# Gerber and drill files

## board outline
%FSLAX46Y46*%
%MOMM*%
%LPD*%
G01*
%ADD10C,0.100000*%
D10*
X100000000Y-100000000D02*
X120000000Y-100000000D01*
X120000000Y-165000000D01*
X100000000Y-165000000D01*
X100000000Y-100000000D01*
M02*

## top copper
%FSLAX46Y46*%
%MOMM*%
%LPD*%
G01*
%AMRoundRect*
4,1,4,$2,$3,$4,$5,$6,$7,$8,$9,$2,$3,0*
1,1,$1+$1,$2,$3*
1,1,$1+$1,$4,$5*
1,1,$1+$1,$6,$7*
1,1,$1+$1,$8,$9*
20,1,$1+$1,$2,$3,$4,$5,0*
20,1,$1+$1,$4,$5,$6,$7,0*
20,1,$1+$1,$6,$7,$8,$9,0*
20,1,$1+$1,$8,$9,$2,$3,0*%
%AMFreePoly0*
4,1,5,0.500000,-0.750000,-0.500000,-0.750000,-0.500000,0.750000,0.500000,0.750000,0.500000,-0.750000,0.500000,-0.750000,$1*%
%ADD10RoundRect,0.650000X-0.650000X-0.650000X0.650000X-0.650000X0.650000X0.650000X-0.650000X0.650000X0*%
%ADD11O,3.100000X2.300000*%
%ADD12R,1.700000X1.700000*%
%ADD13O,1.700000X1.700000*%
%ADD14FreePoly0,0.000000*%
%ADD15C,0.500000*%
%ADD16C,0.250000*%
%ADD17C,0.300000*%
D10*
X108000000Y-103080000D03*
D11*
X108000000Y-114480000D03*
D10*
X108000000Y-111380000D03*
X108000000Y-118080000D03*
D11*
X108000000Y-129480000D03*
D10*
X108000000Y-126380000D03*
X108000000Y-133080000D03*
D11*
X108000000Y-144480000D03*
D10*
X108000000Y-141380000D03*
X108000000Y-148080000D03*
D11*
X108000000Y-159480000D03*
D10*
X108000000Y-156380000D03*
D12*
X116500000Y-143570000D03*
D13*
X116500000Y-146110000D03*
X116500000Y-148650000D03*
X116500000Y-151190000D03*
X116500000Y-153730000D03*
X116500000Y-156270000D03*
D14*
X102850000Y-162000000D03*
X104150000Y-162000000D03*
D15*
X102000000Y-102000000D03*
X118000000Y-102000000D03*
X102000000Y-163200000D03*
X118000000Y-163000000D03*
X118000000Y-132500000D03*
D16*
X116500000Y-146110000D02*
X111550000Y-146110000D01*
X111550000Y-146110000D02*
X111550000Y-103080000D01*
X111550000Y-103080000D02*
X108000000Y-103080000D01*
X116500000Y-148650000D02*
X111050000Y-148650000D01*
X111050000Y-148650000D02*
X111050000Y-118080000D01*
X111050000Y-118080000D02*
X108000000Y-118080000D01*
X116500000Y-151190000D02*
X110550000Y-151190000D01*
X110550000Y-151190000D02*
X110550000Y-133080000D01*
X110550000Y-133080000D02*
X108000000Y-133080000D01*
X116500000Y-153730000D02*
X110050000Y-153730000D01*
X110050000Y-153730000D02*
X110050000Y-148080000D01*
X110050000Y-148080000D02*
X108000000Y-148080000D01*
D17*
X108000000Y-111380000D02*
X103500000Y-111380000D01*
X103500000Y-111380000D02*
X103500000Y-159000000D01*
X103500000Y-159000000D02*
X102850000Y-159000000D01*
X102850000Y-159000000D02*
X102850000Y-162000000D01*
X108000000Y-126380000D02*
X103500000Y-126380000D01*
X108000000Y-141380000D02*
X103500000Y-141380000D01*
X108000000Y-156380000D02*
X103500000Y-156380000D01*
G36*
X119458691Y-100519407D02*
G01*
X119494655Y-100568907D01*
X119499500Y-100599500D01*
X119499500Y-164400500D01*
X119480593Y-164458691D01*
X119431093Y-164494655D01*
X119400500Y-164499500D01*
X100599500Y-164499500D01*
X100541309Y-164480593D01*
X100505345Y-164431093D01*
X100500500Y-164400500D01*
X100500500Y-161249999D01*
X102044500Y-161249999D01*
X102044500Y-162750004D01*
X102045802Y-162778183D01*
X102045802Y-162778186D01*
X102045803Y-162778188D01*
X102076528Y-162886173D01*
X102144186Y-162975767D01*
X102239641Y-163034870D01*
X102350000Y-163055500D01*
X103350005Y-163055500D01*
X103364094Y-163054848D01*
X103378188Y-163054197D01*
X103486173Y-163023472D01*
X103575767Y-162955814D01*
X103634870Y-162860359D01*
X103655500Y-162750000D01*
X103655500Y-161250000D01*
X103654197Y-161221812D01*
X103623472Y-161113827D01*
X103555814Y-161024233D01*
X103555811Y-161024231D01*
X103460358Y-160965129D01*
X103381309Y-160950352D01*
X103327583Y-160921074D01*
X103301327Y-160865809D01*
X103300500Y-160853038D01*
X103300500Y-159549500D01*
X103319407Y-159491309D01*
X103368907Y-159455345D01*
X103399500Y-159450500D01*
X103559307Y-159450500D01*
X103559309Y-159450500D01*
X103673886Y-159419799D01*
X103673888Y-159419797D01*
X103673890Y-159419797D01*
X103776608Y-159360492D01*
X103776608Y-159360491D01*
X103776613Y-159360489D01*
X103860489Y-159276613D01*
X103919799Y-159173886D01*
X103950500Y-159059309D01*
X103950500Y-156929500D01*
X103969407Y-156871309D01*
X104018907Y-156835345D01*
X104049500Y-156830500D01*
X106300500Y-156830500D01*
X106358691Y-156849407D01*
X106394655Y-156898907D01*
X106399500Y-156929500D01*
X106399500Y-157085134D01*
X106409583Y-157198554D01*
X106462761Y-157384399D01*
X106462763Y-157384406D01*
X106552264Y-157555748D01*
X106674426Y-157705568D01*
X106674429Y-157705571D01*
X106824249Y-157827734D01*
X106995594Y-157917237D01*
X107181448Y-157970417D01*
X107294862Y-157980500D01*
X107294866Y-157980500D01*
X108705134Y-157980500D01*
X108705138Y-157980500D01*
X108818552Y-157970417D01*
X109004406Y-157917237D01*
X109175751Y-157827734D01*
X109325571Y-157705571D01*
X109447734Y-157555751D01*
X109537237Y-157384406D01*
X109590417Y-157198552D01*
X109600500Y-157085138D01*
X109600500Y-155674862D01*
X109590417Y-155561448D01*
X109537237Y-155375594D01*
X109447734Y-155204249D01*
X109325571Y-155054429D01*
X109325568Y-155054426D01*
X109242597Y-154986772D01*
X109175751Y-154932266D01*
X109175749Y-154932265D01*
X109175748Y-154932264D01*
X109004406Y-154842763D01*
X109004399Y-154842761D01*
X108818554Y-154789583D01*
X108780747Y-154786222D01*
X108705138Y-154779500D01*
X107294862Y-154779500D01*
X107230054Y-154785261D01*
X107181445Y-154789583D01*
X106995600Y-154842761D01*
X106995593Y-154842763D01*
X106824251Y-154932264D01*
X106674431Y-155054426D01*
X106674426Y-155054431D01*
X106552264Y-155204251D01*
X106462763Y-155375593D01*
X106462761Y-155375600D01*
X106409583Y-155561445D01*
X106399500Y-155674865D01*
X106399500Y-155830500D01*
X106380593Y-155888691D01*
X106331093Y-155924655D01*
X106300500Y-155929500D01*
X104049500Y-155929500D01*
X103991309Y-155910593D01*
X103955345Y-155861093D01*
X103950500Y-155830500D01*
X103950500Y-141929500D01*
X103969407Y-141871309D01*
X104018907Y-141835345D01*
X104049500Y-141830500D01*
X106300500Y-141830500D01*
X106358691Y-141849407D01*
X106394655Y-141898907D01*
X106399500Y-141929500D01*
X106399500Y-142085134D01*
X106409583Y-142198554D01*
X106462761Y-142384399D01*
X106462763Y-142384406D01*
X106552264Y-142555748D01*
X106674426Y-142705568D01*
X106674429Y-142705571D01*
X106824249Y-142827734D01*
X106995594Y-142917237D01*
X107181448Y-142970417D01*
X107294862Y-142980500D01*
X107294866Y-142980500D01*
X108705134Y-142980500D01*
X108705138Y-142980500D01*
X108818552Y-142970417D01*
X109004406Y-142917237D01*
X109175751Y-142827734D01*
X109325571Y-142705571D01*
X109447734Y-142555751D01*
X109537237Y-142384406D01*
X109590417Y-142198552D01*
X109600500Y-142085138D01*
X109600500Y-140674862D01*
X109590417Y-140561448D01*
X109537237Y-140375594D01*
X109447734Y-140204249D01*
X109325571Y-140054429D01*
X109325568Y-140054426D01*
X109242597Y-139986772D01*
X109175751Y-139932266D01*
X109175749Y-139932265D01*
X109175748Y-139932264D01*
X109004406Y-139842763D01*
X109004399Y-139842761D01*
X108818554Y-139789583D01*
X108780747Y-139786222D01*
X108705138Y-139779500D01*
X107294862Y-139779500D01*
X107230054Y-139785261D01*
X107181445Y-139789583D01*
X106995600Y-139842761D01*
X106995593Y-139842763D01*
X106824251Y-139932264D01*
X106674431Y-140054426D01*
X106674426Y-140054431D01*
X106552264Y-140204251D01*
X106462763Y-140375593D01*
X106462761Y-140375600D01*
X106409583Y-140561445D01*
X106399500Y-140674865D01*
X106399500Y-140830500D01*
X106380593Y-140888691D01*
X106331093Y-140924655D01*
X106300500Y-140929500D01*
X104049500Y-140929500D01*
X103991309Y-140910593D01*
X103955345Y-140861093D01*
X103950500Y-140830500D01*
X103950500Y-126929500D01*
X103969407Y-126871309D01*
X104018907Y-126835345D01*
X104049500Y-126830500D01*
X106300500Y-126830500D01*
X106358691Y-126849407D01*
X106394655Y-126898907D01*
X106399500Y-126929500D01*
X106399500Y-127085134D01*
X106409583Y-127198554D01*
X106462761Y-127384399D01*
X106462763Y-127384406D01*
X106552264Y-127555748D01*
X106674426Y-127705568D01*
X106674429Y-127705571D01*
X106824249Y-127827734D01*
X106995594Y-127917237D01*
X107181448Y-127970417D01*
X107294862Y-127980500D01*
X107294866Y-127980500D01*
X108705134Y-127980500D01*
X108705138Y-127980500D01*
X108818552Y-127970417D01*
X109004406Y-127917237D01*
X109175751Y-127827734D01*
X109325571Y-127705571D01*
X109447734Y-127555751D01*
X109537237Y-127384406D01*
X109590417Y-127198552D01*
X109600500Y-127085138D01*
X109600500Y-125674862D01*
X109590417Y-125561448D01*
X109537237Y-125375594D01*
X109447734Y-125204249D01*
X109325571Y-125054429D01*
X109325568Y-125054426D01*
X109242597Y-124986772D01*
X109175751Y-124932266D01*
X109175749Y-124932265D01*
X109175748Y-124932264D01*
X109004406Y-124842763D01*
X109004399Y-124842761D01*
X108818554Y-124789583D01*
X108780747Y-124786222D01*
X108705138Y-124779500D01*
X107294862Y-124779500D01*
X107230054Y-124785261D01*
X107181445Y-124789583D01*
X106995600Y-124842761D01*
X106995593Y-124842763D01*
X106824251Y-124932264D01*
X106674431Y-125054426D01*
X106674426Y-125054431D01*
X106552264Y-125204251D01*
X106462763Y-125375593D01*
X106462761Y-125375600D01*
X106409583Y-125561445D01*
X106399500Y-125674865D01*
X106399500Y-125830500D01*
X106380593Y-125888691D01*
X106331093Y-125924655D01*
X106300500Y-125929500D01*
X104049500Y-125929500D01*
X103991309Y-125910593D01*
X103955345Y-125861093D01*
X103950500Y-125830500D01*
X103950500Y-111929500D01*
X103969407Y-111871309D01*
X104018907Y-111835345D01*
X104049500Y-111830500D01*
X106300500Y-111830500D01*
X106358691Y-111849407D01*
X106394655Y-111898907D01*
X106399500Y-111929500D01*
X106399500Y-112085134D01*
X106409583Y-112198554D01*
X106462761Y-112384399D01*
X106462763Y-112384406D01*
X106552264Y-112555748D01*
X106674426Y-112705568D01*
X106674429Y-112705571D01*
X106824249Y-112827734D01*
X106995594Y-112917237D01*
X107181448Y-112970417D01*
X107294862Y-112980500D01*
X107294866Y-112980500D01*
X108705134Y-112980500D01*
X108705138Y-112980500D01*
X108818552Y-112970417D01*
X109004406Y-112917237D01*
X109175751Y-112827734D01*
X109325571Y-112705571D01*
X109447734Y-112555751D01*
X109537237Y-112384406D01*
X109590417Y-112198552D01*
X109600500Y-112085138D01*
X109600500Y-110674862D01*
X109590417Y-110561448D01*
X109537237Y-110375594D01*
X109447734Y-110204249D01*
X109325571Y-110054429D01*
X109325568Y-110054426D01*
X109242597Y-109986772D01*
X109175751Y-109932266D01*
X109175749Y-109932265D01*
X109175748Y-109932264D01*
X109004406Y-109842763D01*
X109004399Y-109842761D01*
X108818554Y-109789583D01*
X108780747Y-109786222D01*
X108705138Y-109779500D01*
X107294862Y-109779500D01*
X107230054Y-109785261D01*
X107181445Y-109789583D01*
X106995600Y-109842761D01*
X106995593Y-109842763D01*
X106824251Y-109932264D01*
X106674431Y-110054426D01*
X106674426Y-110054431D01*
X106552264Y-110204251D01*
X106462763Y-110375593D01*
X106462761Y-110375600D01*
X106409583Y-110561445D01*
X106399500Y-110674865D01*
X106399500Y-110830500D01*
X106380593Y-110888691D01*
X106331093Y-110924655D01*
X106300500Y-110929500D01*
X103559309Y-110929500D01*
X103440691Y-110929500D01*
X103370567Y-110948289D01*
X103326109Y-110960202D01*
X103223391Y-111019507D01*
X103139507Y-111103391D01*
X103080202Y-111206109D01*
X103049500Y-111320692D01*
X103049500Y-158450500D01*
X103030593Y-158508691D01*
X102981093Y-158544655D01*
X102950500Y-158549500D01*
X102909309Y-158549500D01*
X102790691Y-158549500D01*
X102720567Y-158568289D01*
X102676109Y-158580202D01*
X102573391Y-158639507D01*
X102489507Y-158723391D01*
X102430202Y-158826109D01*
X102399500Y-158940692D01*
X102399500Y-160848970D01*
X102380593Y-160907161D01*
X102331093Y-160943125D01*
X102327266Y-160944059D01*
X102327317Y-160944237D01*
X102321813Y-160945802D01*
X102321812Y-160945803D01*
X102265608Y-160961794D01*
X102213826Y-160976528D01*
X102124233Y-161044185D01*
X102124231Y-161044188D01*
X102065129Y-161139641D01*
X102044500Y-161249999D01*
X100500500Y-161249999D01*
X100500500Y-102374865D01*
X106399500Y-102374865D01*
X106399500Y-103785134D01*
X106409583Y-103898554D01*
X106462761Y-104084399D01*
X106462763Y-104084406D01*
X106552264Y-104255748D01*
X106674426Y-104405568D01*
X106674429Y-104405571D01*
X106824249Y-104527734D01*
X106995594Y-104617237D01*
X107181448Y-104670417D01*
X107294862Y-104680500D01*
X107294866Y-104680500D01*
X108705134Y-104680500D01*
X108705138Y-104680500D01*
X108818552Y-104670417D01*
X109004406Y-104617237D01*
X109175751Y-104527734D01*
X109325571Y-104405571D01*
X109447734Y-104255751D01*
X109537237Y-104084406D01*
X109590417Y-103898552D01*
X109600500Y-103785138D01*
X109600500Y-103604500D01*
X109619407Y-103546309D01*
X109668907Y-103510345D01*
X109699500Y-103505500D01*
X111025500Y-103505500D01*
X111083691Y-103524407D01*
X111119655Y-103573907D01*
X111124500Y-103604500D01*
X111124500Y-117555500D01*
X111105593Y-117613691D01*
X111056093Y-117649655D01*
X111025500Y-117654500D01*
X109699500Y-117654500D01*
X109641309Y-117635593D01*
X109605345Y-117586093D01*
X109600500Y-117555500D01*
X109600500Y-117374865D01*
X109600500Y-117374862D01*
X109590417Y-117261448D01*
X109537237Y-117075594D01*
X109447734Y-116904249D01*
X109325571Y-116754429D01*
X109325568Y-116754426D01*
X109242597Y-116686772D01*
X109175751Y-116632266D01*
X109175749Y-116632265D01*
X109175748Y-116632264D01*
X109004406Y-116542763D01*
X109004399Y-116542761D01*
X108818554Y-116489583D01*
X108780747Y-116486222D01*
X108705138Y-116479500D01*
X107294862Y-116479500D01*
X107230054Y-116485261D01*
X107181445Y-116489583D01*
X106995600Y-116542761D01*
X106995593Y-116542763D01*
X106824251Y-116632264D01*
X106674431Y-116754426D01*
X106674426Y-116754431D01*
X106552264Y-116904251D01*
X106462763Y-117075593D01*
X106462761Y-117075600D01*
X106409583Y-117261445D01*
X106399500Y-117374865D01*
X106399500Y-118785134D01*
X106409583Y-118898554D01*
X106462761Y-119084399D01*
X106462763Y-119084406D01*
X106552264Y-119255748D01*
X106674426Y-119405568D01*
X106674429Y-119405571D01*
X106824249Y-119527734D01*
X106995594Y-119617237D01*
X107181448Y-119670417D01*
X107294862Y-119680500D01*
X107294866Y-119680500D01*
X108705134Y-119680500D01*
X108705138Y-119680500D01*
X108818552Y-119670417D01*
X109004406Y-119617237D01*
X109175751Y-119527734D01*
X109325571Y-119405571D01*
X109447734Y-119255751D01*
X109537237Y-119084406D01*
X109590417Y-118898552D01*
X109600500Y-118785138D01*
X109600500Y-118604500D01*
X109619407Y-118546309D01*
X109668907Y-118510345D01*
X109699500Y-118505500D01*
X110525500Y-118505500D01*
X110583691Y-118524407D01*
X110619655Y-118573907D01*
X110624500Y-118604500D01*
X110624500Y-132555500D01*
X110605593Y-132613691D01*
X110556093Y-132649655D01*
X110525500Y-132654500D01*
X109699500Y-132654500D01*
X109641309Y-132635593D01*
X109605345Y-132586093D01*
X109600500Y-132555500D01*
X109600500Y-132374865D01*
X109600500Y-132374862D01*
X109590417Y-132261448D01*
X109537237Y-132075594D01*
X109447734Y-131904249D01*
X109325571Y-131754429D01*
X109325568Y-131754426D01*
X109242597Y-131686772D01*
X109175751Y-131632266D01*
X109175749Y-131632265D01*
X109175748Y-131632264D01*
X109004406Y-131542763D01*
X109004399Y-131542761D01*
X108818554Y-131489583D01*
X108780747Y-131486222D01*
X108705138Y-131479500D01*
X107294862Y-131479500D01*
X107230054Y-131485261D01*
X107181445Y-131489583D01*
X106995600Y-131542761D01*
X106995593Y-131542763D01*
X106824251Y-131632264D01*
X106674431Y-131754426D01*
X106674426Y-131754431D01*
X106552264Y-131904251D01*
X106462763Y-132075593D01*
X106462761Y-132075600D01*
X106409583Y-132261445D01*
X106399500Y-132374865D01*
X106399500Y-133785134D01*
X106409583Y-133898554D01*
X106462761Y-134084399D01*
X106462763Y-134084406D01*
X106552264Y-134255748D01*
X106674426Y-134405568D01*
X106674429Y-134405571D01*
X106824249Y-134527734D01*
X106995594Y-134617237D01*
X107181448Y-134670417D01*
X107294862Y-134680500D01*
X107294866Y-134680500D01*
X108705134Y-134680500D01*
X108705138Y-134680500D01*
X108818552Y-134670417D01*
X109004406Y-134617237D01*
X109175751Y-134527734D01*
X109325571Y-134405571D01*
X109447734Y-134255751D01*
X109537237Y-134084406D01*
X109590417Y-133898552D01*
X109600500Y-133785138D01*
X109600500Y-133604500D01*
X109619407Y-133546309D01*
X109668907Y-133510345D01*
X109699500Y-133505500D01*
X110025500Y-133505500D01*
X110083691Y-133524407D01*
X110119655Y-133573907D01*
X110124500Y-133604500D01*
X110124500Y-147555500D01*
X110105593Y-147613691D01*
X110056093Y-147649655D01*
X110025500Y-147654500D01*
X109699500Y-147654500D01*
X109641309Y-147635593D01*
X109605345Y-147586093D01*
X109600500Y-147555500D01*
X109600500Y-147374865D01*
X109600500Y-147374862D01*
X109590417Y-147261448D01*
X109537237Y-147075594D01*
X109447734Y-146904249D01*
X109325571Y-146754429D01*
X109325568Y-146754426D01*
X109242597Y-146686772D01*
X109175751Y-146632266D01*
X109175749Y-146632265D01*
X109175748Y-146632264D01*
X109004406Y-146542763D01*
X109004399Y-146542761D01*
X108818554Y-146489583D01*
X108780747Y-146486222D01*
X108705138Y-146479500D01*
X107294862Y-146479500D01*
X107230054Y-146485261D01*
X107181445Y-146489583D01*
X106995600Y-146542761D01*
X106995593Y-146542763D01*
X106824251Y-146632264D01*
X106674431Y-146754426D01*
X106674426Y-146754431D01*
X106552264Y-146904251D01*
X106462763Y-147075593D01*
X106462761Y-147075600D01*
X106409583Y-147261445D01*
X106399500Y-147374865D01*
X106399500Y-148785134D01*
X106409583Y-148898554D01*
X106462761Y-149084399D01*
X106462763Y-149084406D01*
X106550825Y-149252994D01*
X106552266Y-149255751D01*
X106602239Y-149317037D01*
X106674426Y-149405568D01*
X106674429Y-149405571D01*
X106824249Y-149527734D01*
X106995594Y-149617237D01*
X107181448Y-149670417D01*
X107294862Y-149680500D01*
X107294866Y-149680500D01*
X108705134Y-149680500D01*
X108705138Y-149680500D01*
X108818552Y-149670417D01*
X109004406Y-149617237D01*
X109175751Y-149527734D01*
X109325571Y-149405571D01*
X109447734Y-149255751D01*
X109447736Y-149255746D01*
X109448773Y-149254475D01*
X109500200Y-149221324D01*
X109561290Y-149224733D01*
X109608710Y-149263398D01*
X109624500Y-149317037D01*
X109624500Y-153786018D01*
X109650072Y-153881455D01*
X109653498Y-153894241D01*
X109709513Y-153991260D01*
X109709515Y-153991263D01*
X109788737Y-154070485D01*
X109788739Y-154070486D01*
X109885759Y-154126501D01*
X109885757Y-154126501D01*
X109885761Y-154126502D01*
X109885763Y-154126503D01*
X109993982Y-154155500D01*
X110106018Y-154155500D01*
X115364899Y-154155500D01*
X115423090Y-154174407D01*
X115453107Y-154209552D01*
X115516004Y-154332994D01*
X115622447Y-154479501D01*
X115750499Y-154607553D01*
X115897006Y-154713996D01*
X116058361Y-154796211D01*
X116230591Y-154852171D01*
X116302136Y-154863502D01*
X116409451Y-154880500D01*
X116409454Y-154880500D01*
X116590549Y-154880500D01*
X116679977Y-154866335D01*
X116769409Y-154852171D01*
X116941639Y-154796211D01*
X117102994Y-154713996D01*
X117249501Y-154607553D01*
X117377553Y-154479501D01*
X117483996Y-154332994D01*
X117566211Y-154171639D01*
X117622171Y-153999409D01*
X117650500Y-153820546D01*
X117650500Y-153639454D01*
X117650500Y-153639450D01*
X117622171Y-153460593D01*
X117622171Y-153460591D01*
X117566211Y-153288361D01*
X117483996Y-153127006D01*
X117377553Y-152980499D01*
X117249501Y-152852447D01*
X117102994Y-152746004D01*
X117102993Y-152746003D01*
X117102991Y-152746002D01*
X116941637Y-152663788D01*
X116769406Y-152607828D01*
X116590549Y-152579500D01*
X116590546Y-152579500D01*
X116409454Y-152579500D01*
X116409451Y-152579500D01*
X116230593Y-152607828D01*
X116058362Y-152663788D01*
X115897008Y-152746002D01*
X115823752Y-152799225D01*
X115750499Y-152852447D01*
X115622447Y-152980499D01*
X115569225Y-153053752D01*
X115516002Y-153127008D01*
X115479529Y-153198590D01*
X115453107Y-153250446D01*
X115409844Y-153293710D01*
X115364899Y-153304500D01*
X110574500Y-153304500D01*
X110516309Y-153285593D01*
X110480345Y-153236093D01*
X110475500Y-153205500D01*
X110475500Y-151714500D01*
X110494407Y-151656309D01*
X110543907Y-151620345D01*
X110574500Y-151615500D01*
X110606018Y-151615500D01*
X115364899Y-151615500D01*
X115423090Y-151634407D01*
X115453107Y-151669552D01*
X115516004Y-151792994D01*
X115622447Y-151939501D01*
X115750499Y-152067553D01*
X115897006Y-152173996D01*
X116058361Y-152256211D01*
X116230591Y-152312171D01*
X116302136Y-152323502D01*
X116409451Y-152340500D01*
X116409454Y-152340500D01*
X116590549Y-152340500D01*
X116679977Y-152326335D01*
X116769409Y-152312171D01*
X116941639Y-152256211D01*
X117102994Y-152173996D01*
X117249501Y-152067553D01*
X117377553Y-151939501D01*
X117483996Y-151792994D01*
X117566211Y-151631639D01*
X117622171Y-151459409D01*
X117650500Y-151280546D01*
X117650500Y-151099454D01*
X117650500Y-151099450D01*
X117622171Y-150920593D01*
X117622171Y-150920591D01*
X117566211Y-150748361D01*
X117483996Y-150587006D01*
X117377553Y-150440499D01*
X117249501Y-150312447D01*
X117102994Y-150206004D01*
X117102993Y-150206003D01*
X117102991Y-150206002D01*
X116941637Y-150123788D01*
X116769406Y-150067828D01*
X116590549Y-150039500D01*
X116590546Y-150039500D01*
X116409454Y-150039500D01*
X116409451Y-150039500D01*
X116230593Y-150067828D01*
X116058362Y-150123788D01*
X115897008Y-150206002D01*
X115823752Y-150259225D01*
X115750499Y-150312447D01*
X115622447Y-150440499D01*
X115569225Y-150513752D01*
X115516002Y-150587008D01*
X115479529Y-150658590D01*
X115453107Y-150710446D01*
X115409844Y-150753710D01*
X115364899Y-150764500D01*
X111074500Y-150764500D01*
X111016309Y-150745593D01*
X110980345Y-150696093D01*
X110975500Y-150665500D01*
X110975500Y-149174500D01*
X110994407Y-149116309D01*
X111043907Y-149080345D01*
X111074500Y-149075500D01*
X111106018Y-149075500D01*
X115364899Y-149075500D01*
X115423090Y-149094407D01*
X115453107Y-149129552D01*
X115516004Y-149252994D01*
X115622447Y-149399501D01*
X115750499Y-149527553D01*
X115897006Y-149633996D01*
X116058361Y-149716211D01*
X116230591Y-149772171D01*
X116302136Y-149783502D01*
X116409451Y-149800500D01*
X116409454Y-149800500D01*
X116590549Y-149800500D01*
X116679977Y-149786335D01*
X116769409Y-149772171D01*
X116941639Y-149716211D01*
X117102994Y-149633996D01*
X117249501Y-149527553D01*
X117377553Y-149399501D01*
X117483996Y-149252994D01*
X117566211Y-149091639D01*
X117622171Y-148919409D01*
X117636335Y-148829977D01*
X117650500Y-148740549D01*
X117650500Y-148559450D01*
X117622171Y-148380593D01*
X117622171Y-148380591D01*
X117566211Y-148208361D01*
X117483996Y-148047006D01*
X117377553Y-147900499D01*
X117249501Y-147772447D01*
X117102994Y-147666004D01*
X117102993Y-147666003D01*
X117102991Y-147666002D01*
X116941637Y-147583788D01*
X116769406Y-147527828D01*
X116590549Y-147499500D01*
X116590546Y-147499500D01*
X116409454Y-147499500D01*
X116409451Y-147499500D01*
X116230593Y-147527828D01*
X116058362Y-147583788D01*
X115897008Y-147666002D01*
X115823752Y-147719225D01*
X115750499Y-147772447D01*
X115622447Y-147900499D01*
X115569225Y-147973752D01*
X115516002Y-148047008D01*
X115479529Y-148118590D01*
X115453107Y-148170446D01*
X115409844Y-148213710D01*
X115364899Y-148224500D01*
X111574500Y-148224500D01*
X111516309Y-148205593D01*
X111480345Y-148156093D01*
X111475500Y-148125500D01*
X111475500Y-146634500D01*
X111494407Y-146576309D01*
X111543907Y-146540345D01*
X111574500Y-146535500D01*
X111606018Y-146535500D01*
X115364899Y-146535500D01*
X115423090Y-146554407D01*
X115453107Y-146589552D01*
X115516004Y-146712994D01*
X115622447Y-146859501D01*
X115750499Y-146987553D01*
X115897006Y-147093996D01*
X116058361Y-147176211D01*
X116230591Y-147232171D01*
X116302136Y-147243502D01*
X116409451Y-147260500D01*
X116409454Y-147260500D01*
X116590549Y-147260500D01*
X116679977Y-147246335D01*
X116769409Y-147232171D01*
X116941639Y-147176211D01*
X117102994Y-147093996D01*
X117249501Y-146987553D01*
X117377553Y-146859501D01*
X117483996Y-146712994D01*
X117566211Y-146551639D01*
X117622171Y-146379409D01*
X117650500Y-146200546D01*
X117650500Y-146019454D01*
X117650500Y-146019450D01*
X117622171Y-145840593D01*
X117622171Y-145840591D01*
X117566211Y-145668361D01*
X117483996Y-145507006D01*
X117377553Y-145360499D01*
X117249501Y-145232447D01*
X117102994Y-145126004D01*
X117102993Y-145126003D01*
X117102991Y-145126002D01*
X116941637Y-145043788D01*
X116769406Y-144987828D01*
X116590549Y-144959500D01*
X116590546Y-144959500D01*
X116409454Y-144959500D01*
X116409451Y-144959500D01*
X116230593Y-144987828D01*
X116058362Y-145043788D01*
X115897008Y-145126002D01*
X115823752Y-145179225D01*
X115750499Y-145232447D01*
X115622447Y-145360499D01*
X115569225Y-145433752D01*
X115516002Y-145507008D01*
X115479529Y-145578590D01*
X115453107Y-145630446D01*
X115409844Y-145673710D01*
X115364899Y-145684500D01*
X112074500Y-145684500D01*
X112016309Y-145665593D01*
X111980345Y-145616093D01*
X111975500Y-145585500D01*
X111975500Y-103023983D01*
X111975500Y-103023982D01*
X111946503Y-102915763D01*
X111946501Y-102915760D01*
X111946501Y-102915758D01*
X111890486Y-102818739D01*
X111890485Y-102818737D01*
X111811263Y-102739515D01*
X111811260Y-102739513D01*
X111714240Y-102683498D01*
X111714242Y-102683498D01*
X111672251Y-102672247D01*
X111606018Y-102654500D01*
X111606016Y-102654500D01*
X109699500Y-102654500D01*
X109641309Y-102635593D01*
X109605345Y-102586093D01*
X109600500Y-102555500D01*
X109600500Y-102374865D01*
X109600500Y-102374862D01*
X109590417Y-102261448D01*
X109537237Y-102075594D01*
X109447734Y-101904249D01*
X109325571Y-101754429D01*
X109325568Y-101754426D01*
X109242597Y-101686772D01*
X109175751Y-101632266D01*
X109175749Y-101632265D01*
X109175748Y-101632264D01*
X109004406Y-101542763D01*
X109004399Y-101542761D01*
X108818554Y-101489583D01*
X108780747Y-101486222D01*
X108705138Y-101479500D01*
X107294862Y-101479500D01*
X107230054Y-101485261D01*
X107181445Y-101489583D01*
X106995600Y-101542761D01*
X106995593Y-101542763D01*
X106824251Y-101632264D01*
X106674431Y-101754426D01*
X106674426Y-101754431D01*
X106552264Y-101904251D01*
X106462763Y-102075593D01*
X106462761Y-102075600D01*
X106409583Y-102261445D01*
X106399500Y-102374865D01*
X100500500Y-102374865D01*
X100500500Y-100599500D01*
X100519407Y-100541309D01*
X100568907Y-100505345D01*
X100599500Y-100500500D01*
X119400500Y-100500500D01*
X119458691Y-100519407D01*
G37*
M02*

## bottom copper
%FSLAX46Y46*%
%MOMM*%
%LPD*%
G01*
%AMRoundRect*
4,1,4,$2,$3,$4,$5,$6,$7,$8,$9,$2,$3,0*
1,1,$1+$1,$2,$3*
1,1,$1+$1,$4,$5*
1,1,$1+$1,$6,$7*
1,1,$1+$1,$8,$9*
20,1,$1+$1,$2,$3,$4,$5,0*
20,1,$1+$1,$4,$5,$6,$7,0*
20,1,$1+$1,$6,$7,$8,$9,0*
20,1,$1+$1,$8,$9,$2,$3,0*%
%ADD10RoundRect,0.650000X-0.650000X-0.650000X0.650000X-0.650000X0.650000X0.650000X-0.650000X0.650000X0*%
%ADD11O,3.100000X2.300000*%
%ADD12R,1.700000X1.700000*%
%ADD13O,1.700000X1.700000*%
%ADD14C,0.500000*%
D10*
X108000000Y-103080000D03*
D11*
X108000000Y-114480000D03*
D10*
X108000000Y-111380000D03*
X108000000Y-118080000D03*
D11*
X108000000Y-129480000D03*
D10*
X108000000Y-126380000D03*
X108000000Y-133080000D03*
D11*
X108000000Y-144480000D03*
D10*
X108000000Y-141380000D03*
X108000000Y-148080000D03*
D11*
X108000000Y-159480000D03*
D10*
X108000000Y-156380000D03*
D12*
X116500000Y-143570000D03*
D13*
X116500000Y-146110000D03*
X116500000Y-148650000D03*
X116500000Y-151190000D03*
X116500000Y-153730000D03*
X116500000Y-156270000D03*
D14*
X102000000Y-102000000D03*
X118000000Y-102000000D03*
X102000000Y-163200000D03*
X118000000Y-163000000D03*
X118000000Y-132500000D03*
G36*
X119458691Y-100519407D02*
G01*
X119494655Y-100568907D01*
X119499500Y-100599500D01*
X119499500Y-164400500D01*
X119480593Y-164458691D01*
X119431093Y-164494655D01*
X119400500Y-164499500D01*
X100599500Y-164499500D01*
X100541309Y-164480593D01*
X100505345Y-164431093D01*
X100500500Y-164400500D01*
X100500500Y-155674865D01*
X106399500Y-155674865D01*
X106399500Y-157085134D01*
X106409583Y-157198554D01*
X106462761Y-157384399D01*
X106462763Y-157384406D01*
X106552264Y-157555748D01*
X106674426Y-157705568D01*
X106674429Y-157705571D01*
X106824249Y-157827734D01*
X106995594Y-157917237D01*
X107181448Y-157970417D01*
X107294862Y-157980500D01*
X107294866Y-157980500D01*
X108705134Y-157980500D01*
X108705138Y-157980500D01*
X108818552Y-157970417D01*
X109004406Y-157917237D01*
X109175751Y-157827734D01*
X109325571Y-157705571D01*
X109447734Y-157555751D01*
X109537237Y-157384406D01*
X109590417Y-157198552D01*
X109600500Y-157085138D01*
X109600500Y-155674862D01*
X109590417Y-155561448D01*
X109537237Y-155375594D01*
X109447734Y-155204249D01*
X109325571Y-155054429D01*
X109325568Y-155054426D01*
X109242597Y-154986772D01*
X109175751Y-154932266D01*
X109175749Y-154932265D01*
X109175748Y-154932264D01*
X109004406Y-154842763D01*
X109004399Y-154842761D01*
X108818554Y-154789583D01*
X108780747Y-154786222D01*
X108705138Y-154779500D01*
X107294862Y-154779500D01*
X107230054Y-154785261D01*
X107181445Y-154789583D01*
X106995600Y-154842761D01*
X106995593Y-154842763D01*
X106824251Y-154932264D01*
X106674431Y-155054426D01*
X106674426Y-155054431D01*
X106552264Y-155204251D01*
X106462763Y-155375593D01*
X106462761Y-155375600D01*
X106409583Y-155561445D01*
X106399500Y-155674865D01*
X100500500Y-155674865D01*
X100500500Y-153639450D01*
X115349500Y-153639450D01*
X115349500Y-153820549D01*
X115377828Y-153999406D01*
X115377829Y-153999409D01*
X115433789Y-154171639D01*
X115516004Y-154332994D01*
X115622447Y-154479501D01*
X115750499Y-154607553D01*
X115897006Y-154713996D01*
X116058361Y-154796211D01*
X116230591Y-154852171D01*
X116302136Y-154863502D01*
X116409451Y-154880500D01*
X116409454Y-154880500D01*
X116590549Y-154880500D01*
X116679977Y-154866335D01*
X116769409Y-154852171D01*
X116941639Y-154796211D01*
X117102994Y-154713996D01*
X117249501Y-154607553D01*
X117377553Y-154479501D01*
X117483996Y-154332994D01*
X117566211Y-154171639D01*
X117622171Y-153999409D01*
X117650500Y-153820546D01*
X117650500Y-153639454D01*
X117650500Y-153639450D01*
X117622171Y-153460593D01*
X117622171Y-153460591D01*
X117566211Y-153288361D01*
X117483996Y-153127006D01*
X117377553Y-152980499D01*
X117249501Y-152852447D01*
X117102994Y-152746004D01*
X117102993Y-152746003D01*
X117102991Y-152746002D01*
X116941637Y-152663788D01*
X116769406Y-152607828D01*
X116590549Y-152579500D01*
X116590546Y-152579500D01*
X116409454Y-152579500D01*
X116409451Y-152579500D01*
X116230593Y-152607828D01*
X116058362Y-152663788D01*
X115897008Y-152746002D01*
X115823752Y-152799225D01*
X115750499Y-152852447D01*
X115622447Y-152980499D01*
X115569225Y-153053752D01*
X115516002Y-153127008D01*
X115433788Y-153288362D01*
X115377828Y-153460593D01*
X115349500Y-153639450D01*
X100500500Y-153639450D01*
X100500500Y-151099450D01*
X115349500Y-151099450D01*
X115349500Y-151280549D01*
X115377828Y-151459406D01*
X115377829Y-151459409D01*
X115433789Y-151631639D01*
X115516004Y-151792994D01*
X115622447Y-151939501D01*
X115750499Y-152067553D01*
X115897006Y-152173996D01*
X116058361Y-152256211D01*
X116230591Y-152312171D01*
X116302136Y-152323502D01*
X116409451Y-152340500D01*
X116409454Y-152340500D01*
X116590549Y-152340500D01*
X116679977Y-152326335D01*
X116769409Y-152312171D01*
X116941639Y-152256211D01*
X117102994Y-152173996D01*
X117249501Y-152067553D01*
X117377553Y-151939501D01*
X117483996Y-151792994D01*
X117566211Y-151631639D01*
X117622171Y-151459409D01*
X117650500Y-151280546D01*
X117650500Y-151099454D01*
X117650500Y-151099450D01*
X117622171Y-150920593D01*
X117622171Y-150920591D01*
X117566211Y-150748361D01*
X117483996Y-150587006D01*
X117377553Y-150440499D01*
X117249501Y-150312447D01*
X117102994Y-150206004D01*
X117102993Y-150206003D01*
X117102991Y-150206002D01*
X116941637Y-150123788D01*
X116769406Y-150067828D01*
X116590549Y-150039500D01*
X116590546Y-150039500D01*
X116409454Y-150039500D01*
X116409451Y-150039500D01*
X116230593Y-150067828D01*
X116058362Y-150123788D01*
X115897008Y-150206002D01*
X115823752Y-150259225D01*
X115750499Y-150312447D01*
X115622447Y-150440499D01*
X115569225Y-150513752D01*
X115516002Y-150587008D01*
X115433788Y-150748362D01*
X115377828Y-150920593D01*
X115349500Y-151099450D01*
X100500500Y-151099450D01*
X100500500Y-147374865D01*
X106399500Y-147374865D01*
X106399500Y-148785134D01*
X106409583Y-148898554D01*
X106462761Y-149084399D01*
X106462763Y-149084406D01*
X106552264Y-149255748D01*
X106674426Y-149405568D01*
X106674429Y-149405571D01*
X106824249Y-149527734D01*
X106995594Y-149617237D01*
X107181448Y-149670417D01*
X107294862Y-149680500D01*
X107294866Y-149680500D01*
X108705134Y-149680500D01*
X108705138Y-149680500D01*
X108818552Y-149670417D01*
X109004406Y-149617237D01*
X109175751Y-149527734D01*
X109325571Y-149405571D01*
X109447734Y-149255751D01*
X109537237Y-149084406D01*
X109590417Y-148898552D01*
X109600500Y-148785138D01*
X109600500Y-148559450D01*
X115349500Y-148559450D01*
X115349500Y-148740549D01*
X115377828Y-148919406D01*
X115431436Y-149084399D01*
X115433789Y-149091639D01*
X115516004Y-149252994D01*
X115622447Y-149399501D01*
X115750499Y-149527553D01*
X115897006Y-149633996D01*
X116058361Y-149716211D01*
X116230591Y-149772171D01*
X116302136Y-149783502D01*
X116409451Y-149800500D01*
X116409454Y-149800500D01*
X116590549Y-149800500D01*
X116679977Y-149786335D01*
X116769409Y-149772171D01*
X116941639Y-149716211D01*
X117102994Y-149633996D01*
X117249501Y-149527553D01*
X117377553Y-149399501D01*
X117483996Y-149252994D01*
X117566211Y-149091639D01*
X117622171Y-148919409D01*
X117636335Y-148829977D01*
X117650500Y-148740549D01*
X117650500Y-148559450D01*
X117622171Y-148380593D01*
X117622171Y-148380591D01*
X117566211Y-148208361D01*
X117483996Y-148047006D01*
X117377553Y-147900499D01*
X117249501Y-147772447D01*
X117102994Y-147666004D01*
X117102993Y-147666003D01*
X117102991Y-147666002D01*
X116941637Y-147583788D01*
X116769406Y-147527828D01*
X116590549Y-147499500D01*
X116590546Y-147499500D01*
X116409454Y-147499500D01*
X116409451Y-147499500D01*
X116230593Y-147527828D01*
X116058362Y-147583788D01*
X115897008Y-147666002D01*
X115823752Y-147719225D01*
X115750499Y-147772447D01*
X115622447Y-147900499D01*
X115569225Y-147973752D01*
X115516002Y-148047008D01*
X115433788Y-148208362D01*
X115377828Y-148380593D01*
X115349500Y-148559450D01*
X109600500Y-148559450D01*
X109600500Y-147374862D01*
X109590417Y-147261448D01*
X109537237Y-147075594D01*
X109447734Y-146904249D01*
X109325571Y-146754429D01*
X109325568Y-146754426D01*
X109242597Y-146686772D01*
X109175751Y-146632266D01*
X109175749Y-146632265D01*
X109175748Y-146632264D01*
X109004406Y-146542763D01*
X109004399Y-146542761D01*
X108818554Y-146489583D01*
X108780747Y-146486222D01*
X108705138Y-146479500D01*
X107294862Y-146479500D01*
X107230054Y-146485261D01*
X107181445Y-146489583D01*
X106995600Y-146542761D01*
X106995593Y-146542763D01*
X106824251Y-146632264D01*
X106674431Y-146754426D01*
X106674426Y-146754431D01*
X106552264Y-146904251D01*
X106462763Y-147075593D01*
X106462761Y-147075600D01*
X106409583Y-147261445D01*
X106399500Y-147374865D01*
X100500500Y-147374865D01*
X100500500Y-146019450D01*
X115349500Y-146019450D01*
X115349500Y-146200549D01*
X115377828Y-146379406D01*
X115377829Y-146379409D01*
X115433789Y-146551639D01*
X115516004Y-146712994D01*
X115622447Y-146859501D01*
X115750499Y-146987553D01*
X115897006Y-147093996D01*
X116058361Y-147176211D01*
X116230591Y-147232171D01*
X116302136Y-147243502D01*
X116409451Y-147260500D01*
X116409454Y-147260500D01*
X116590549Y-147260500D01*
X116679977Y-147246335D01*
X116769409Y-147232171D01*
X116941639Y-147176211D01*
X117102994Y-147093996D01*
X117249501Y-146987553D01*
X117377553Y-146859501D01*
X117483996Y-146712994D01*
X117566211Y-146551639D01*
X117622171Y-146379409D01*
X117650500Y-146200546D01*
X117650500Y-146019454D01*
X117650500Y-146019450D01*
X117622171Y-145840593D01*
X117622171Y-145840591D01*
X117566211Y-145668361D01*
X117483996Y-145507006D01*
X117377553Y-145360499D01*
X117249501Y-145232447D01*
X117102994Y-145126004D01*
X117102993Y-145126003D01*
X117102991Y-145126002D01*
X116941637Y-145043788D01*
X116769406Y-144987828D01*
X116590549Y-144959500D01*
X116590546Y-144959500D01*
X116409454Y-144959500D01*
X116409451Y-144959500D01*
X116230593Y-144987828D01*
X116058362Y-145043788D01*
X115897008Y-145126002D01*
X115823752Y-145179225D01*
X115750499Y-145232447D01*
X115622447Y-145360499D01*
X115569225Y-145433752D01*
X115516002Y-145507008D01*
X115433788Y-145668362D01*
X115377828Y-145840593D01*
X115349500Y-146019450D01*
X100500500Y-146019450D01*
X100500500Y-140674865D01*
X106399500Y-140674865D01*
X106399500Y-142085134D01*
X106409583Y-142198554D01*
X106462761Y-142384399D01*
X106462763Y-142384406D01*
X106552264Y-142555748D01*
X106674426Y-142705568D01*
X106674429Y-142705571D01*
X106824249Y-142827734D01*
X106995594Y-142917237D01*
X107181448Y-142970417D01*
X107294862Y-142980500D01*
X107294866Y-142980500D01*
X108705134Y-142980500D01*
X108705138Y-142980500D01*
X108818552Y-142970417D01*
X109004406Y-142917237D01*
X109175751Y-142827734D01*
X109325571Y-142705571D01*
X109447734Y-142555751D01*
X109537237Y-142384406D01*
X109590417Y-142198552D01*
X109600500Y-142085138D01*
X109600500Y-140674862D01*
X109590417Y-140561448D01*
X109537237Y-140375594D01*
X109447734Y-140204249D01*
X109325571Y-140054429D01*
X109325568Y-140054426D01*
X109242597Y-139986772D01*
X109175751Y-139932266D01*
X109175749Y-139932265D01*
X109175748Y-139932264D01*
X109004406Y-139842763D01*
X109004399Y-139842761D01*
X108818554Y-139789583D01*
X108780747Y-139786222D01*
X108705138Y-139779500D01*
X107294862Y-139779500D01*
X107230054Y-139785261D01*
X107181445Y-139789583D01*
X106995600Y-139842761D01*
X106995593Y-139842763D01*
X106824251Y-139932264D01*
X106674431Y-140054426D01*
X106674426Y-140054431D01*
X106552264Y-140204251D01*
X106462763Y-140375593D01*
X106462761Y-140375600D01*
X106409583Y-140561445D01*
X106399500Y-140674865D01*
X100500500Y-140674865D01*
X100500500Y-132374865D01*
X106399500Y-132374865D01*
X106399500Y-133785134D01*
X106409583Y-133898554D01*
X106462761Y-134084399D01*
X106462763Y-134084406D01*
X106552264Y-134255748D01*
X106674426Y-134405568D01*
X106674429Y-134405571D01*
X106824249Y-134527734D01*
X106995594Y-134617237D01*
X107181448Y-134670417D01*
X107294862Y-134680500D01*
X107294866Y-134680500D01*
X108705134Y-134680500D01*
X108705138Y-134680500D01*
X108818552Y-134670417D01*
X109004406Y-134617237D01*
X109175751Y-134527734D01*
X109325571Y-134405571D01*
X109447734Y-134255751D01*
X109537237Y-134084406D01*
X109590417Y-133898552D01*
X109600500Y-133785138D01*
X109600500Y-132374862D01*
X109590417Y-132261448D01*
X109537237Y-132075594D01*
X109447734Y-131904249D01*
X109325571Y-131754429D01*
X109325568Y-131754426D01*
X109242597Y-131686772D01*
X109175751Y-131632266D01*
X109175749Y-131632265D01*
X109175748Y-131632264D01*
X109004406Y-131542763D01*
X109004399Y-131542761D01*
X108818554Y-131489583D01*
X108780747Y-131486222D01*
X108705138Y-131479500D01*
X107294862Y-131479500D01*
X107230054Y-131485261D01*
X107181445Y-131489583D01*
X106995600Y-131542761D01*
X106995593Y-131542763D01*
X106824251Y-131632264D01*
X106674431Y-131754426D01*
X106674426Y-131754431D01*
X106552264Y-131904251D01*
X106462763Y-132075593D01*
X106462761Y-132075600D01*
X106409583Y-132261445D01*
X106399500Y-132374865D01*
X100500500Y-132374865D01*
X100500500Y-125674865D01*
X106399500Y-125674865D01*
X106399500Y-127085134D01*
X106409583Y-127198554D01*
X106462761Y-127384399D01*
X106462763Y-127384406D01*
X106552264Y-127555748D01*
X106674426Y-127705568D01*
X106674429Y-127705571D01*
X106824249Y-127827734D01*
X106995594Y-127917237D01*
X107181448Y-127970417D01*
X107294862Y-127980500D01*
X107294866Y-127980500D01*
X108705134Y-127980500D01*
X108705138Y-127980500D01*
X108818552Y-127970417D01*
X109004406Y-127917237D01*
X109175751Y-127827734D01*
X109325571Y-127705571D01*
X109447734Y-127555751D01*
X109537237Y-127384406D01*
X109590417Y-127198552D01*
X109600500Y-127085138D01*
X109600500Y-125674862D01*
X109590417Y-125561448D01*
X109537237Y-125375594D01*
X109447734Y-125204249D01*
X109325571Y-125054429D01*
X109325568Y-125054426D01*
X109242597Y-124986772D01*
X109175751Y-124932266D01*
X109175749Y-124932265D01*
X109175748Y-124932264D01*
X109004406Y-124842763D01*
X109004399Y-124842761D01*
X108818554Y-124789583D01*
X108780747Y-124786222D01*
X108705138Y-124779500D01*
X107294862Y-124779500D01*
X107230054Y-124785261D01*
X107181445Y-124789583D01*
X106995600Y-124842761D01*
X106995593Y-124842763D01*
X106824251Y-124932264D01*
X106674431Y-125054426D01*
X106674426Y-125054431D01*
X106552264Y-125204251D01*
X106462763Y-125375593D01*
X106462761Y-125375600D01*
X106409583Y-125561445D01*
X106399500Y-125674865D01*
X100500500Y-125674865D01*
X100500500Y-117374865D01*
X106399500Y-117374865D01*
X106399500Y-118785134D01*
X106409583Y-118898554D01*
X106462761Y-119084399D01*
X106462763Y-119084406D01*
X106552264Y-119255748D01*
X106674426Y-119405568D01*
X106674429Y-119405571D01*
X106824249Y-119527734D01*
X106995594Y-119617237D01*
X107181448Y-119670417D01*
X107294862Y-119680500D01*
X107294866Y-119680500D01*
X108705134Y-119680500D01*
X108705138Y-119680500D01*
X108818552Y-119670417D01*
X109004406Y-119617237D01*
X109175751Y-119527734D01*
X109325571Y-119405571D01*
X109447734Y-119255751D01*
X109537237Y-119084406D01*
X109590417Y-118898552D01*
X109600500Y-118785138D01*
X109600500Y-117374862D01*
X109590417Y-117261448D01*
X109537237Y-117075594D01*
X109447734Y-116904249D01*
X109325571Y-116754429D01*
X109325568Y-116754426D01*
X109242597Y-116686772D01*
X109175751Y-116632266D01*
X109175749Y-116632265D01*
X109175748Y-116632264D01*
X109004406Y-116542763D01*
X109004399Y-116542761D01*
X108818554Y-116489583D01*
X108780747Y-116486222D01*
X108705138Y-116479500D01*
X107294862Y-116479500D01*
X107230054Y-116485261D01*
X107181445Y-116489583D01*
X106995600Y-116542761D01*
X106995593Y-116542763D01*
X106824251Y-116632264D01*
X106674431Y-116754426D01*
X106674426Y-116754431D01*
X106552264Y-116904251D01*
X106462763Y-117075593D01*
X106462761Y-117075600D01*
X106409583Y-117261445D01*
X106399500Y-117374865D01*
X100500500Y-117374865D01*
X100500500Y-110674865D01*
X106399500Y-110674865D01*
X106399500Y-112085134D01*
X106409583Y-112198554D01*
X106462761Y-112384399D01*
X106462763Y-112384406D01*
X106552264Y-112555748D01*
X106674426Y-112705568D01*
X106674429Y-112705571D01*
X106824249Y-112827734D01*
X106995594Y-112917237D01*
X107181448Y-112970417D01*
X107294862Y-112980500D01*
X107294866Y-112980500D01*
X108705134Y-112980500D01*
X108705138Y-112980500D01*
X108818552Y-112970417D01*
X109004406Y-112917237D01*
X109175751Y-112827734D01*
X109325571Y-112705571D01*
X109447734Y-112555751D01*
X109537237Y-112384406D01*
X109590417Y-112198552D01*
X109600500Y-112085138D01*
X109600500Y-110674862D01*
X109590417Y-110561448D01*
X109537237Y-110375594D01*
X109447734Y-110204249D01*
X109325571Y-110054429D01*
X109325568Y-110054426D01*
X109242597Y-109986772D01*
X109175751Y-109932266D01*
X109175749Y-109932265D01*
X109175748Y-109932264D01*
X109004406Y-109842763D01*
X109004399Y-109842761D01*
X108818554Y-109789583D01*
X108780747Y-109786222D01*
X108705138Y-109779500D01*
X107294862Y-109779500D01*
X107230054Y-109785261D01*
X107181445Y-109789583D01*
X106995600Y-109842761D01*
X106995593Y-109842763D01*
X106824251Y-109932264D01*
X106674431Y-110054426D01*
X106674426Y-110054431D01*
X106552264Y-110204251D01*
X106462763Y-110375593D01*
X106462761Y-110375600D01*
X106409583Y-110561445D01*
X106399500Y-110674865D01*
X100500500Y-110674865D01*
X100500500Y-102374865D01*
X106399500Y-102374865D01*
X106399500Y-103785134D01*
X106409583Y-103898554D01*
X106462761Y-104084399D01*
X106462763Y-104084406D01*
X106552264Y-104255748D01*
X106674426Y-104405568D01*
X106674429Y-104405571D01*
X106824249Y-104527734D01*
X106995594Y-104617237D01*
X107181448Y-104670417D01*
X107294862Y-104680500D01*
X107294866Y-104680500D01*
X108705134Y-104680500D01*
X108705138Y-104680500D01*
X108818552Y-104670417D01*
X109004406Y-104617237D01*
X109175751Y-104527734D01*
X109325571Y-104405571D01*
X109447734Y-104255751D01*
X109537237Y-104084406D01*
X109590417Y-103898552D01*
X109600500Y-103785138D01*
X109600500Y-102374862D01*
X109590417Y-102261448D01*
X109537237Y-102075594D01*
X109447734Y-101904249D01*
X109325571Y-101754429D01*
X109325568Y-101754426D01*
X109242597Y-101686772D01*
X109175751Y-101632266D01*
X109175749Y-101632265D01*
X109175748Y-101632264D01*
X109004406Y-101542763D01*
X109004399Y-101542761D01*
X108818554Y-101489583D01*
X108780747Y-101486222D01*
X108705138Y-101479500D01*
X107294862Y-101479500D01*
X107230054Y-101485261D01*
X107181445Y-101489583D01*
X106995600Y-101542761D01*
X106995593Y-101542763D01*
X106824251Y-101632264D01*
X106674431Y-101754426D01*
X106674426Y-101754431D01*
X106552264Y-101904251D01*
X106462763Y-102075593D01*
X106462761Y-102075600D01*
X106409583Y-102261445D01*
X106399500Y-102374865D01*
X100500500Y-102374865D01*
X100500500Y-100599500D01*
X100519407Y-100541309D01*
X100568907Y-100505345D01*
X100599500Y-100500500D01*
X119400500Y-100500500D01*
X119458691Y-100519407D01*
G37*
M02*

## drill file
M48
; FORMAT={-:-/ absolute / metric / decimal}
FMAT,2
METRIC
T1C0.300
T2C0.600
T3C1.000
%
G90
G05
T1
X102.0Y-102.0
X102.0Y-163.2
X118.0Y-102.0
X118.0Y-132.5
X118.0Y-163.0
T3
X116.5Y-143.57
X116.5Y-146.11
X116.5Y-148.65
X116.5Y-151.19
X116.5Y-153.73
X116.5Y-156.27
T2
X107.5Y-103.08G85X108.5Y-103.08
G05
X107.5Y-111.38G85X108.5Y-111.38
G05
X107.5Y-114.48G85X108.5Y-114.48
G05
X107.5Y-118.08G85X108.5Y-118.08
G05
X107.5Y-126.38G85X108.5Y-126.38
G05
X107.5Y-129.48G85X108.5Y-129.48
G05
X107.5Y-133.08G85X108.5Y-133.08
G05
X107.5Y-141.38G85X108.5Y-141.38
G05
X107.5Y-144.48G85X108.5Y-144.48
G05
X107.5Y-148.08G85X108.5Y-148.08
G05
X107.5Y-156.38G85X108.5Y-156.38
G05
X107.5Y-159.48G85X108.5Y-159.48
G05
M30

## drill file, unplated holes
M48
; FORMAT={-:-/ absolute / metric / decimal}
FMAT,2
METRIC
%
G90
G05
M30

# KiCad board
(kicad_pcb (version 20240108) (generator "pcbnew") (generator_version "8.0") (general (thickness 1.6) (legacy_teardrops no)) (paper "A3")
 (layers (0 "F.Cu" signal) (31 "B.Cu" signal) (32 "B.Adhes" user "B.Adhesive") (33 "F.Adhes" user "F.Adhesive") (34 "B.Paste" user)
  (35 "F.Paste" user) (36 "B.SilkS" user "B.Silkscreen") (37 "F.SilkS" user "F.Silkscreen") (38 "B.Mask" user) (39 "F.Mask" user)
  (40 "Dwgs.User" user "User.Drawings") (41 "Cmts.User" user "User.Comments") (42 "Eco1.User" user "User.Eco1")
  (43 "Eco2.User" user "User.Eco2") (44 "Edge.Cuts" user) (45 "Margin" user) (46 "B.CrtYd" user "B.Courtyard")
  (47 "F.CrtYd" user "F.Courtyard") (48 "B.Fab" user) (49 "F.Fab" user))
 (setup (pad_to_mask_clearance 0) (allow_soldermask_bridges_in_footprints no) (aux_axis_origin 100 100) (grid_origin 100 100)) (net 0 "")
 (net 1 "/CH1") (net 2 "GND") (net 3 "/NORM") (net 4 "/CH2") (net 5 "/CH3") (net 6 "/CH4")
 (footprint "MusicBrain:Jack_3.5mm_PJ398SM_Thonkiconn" (layer "F.Cu") (at 108 108)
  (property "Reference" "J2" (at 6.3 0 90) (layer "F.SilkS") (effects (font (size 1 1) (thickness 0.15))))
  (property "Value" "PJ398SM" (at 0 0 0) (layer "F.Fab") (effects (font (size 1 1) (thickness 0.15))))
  (pad "1" thru_hole roundrect (at 0 -4.92) (size 2.6 2.6) (drill oval 1.6 0.6) (layers "*.Cu" "*.Mask") (roundrect_rratio 0.25)
   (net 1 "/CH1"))
  (pad "2" thru_hole oval (at 0 6.48) (size 3.1 2.3) (drill oval 1.6 0.6) (layers "*.Cu" "*.Mask") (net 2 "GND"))
  (pad "3" thru_hole roundrect (at 0 3.38) (size 2.6 2.6) (drill oval 1.6 0.6) (layers "*.Cu" "*.Mask") (roundrect_rratio 0.25)
   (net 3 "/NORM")))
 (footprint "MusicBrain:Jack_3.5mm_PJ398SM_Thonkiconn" (layer "F.Cu") (at 108 123)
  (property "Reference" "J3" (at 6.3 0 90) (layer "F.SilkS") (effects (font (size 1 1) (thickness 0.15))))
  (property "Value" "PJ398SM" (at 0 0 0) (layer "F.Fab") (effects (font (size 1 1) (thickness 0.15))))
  (pad "1" thru_hole roundrect (at 0 -4.92) (size 2.6 2.6) (drill oval 1.6 0.6) (layers "*.Cu" "*.Mask") (roundrect_rratio 0.25)
   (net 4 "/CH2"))
  (pad "2" thru_hole oval (at 0 6.48) (size 3.1 2.3) (drill oval 1.6 0.6) (layers "*.Cu" "*.Mask") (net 2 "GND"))
  (pad "3" thru_hole roundrect (at 0 3.38) (size 2.6 2.6) (drill oval 1.6 0.6) (layers "*.Cu" "*.Mask") (roundrect_rratio 0.25)
   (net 3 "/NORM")))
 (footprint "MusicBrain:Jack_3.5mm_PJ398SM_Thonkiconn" (layer "F.Cu") (at 108 138)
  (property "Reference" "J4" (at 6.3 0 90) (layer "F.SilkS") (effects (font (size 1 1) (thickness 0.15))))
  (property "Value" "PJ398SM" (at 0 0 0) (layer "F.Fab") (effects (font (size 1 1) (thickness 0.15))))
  (pad "1" thru_hole roundrect (at 0 -4.92) (size 2.6 2.6) (drill oval 1.6 0.6) (layers "*.Cu" "*.Mask") (roundrect_rratio 0.25)
   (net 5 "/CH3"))
  (pad "2" thru_hole oval (at 0 6.48) (size 3.1 2.3) (drill oval 1.6 0.6) (layers "*.Cu" "*.Mask") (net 2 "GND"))
  (pad "3" thru_hole roundrect (at 0 3.38) (size 2.6 2.6) (drill oval 1.6 0.6) (layers "*.Cu" "*.Mask") (roundrect_rratio 0.25)
   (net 3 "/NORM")))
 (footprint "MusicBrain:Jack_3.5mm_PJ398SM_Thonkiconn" (layer "F.Cu") (at 108 153)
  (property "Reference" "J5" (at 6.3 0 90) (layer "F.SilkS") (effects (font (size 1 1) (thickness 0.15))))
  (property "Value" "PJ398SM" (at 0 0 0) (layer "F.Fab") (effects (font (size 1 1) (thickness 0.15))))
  (pad "1" thru_hole roundrect (at 0 -4.92) (size 2.6 2.6) (drill oval 1.6 0.6) (layers "*.Cu" "*.Mask") (roundrect_rratio 0.25)
   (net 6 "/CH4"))
  (pad "2" thru_hole oval (at 0 6.48) (size 3.1 2.3) (drill oval 1.6 0.6) (layers "*.Cu" "*.Mask") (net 2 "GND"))
  (pad "3" thru_hole roundrect (at 0 3.38) (size 2.6 2.6) (drill oval 1.6 0.6) (layers "*.Cu" "*.Mask") (roundrect_rratio 0.25)
   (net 3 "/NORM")))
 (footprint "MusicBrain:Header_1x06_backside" (layer "B.Cu") (at 116.5 143.57 180)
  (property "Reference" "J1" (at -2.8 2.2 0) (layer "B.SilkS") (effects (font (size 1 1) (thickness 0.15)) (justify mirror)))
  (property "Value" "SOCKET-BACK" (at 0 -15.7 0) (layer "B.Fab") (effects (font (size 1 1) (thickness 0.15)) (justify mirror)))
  (pad "1" thru_hole rect (at 0 -0 180) (size 1.7 1.7) (drill 1.0) (layers "*.Cu" "*.Mask") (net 2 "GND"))
  (pad "2" thru_hole oval (at 0 -2.54 180) (size 1.7 1.7) (drill 1.0) (layers "*.Cu" "*.Mask") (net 1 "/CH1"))
  (pad "3" thru_hole oval (at 0 -5.08 180) (size 1.7 1.7) (drill 1.0) (layers "*.Cu" "*.Mask") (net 4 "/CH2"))
  (pad "4" thru_hole oval (at 0 -7.62 180) (size 1.7 1.7) (drill 1.0) (layers "*.Cu" "*.Mask") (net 5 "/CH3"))
  (pad "5" thru_hole oval (at 0 -10.16 180) (size 1.7 1.7) (drill 1.0) (layers "*.Cu" "*.Mask") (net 6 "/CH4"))
  (pad "6" thru_hole oval (at 0 -12.7 180) (size 1.7 1.7) (drill 1.0) (layers "*.Cu" "*.Mask") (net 2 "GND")))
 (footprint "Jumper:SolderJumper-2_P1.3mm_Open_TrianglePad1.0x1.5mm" (layer "F.Cu") (at 103.5 162)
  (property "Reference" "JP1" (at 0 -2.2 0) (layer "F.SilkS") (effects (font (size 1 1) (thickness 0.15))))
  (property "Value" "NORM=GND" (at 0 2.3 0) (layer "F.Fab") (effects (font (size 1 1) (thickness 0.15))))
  (pad "1" smd custom (at -0.65 0) (size 1 1.5) (layers "F.Cu" "F.Mask") (options (clearance outline) (anchor rect)) (primitives)
   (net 3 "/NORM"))
  (pad "2" smd custom (at 0.65 0) (size 1 1.5) (layers "F.Cu" "F.Mask") (options (clearance outline) (anchor rect)) (primitives)
   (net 2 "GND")))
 (segment (start 116.5 146.11) (end 111.55 146.11) (width 0.25) (layer "F.Cu") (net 1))
 (segment (start 111.55 146.11) (end 111.55 103.08) (width 0.25) (layer "F.Cu") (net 1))
 (segment (start 111.55 103.08) (end 108 103.08) (width 0.25) (layer "F.Cu") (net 1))
 (segment (start 116.5 148.65) (end 111.05 148.65) (width 0.25) (layer "F.Cu") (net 4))
 (segment (start 111.05 148.65) (end 111.05 118.08) (width 0.25) (layer "F.Cu") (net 4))
 (segment (start 111.05 118.08) (end 108 118.08) (width 0.25) (layer "F.Cu") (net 4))
 (segment (start 116.5 151.19) (end 110.55 151.19) (width 0.25) (layer "F.Cu") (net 5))
 (segment (start 110.55 151.19) (end 110.55 133.08) (width 0.25) (layer "F.Cu") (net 5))
 (segment (start 110.55 133.08) (end 108 133.08) (width 0.25) (layer "F.Cu") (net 5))
 (segment (start 116.5 153.73) (end 110.05 153.73) (width 0.25) (layer "F.Cu") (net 6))
 (segment (start 110.05 153.73) (end 110.05 148.08) (width 0.25) (layer "F.Cu") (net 6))
 (segment (start 110.05 148.08) (end 108 148.08) (width 0.25) (layer "F.Cu") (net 6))
 (segment (start 108 111.38) (end 103.5 111.38) (width 0.3) (layer "F.Cu") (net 3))
 (segment (start 103.5 111.38) (end 103.5 159) (width 0.3) (layer "F.Cu") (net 3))
 (segment (start 103.5 159) (end 102.85 159) (width 0.3) (layer "F.Cu") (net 3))
 (segment (start 102.85 159) (end 102.85 162) (width 0.3) (layer "F.Cu") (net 3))
 (segment (start 108 126.38) (end 103.5 126.38) (width 0.3) (layer "F.Cu") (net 3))
 (segment (start 108 141.38) (end 103.5 141.38) (width 0.3) (layer "F.Cu") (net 3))
 (segment (start 108 156.38) (end 103.5 156.38) (width 0.3) (layer "F.Cu") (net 3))
 (via (at 102 102) (size 0.5) (drill 0.3) (layers "F.Cu" "B.Cu") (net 2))
 (via (at 118 102) (size 0.5) (drill 0.3) (layers "F.Cu" "B.Cu") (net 2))
 (via (at 102 163.2) (size 0.5) (drill 0.3) (layers "F.Cu" "B.Cu") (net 2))
 (via (at 118 163) (size 0.5) (drill 0.3) (layers "F.Cu" "B.Cu") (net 2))
 (via (at 118 132.5) (size 0.5) (drill 0.3) (layers "F.Cu" "B.Cu") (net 2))
 (gr_rect (start 100 100) (end 120 165) (stroke (width 0.1) (type default)) (fill none) (layer "Edge.Cuts"))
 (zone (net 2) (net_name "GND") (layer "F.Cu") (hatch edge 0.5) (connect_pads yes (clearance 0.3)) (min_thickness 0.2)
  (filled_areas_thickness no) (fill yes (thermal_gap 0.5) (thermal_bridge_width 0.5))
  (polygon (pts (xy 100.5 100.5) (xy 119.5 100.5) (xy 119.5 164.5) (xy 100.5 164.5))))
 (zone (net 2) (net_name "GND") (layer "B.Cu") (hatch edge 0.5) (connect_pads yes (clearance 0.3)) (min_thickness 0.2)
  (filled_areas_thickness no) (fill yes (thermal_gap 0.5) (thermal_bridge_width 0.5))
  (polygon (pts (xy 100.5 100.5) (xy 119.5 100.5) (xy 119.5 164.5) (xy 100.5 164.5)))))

